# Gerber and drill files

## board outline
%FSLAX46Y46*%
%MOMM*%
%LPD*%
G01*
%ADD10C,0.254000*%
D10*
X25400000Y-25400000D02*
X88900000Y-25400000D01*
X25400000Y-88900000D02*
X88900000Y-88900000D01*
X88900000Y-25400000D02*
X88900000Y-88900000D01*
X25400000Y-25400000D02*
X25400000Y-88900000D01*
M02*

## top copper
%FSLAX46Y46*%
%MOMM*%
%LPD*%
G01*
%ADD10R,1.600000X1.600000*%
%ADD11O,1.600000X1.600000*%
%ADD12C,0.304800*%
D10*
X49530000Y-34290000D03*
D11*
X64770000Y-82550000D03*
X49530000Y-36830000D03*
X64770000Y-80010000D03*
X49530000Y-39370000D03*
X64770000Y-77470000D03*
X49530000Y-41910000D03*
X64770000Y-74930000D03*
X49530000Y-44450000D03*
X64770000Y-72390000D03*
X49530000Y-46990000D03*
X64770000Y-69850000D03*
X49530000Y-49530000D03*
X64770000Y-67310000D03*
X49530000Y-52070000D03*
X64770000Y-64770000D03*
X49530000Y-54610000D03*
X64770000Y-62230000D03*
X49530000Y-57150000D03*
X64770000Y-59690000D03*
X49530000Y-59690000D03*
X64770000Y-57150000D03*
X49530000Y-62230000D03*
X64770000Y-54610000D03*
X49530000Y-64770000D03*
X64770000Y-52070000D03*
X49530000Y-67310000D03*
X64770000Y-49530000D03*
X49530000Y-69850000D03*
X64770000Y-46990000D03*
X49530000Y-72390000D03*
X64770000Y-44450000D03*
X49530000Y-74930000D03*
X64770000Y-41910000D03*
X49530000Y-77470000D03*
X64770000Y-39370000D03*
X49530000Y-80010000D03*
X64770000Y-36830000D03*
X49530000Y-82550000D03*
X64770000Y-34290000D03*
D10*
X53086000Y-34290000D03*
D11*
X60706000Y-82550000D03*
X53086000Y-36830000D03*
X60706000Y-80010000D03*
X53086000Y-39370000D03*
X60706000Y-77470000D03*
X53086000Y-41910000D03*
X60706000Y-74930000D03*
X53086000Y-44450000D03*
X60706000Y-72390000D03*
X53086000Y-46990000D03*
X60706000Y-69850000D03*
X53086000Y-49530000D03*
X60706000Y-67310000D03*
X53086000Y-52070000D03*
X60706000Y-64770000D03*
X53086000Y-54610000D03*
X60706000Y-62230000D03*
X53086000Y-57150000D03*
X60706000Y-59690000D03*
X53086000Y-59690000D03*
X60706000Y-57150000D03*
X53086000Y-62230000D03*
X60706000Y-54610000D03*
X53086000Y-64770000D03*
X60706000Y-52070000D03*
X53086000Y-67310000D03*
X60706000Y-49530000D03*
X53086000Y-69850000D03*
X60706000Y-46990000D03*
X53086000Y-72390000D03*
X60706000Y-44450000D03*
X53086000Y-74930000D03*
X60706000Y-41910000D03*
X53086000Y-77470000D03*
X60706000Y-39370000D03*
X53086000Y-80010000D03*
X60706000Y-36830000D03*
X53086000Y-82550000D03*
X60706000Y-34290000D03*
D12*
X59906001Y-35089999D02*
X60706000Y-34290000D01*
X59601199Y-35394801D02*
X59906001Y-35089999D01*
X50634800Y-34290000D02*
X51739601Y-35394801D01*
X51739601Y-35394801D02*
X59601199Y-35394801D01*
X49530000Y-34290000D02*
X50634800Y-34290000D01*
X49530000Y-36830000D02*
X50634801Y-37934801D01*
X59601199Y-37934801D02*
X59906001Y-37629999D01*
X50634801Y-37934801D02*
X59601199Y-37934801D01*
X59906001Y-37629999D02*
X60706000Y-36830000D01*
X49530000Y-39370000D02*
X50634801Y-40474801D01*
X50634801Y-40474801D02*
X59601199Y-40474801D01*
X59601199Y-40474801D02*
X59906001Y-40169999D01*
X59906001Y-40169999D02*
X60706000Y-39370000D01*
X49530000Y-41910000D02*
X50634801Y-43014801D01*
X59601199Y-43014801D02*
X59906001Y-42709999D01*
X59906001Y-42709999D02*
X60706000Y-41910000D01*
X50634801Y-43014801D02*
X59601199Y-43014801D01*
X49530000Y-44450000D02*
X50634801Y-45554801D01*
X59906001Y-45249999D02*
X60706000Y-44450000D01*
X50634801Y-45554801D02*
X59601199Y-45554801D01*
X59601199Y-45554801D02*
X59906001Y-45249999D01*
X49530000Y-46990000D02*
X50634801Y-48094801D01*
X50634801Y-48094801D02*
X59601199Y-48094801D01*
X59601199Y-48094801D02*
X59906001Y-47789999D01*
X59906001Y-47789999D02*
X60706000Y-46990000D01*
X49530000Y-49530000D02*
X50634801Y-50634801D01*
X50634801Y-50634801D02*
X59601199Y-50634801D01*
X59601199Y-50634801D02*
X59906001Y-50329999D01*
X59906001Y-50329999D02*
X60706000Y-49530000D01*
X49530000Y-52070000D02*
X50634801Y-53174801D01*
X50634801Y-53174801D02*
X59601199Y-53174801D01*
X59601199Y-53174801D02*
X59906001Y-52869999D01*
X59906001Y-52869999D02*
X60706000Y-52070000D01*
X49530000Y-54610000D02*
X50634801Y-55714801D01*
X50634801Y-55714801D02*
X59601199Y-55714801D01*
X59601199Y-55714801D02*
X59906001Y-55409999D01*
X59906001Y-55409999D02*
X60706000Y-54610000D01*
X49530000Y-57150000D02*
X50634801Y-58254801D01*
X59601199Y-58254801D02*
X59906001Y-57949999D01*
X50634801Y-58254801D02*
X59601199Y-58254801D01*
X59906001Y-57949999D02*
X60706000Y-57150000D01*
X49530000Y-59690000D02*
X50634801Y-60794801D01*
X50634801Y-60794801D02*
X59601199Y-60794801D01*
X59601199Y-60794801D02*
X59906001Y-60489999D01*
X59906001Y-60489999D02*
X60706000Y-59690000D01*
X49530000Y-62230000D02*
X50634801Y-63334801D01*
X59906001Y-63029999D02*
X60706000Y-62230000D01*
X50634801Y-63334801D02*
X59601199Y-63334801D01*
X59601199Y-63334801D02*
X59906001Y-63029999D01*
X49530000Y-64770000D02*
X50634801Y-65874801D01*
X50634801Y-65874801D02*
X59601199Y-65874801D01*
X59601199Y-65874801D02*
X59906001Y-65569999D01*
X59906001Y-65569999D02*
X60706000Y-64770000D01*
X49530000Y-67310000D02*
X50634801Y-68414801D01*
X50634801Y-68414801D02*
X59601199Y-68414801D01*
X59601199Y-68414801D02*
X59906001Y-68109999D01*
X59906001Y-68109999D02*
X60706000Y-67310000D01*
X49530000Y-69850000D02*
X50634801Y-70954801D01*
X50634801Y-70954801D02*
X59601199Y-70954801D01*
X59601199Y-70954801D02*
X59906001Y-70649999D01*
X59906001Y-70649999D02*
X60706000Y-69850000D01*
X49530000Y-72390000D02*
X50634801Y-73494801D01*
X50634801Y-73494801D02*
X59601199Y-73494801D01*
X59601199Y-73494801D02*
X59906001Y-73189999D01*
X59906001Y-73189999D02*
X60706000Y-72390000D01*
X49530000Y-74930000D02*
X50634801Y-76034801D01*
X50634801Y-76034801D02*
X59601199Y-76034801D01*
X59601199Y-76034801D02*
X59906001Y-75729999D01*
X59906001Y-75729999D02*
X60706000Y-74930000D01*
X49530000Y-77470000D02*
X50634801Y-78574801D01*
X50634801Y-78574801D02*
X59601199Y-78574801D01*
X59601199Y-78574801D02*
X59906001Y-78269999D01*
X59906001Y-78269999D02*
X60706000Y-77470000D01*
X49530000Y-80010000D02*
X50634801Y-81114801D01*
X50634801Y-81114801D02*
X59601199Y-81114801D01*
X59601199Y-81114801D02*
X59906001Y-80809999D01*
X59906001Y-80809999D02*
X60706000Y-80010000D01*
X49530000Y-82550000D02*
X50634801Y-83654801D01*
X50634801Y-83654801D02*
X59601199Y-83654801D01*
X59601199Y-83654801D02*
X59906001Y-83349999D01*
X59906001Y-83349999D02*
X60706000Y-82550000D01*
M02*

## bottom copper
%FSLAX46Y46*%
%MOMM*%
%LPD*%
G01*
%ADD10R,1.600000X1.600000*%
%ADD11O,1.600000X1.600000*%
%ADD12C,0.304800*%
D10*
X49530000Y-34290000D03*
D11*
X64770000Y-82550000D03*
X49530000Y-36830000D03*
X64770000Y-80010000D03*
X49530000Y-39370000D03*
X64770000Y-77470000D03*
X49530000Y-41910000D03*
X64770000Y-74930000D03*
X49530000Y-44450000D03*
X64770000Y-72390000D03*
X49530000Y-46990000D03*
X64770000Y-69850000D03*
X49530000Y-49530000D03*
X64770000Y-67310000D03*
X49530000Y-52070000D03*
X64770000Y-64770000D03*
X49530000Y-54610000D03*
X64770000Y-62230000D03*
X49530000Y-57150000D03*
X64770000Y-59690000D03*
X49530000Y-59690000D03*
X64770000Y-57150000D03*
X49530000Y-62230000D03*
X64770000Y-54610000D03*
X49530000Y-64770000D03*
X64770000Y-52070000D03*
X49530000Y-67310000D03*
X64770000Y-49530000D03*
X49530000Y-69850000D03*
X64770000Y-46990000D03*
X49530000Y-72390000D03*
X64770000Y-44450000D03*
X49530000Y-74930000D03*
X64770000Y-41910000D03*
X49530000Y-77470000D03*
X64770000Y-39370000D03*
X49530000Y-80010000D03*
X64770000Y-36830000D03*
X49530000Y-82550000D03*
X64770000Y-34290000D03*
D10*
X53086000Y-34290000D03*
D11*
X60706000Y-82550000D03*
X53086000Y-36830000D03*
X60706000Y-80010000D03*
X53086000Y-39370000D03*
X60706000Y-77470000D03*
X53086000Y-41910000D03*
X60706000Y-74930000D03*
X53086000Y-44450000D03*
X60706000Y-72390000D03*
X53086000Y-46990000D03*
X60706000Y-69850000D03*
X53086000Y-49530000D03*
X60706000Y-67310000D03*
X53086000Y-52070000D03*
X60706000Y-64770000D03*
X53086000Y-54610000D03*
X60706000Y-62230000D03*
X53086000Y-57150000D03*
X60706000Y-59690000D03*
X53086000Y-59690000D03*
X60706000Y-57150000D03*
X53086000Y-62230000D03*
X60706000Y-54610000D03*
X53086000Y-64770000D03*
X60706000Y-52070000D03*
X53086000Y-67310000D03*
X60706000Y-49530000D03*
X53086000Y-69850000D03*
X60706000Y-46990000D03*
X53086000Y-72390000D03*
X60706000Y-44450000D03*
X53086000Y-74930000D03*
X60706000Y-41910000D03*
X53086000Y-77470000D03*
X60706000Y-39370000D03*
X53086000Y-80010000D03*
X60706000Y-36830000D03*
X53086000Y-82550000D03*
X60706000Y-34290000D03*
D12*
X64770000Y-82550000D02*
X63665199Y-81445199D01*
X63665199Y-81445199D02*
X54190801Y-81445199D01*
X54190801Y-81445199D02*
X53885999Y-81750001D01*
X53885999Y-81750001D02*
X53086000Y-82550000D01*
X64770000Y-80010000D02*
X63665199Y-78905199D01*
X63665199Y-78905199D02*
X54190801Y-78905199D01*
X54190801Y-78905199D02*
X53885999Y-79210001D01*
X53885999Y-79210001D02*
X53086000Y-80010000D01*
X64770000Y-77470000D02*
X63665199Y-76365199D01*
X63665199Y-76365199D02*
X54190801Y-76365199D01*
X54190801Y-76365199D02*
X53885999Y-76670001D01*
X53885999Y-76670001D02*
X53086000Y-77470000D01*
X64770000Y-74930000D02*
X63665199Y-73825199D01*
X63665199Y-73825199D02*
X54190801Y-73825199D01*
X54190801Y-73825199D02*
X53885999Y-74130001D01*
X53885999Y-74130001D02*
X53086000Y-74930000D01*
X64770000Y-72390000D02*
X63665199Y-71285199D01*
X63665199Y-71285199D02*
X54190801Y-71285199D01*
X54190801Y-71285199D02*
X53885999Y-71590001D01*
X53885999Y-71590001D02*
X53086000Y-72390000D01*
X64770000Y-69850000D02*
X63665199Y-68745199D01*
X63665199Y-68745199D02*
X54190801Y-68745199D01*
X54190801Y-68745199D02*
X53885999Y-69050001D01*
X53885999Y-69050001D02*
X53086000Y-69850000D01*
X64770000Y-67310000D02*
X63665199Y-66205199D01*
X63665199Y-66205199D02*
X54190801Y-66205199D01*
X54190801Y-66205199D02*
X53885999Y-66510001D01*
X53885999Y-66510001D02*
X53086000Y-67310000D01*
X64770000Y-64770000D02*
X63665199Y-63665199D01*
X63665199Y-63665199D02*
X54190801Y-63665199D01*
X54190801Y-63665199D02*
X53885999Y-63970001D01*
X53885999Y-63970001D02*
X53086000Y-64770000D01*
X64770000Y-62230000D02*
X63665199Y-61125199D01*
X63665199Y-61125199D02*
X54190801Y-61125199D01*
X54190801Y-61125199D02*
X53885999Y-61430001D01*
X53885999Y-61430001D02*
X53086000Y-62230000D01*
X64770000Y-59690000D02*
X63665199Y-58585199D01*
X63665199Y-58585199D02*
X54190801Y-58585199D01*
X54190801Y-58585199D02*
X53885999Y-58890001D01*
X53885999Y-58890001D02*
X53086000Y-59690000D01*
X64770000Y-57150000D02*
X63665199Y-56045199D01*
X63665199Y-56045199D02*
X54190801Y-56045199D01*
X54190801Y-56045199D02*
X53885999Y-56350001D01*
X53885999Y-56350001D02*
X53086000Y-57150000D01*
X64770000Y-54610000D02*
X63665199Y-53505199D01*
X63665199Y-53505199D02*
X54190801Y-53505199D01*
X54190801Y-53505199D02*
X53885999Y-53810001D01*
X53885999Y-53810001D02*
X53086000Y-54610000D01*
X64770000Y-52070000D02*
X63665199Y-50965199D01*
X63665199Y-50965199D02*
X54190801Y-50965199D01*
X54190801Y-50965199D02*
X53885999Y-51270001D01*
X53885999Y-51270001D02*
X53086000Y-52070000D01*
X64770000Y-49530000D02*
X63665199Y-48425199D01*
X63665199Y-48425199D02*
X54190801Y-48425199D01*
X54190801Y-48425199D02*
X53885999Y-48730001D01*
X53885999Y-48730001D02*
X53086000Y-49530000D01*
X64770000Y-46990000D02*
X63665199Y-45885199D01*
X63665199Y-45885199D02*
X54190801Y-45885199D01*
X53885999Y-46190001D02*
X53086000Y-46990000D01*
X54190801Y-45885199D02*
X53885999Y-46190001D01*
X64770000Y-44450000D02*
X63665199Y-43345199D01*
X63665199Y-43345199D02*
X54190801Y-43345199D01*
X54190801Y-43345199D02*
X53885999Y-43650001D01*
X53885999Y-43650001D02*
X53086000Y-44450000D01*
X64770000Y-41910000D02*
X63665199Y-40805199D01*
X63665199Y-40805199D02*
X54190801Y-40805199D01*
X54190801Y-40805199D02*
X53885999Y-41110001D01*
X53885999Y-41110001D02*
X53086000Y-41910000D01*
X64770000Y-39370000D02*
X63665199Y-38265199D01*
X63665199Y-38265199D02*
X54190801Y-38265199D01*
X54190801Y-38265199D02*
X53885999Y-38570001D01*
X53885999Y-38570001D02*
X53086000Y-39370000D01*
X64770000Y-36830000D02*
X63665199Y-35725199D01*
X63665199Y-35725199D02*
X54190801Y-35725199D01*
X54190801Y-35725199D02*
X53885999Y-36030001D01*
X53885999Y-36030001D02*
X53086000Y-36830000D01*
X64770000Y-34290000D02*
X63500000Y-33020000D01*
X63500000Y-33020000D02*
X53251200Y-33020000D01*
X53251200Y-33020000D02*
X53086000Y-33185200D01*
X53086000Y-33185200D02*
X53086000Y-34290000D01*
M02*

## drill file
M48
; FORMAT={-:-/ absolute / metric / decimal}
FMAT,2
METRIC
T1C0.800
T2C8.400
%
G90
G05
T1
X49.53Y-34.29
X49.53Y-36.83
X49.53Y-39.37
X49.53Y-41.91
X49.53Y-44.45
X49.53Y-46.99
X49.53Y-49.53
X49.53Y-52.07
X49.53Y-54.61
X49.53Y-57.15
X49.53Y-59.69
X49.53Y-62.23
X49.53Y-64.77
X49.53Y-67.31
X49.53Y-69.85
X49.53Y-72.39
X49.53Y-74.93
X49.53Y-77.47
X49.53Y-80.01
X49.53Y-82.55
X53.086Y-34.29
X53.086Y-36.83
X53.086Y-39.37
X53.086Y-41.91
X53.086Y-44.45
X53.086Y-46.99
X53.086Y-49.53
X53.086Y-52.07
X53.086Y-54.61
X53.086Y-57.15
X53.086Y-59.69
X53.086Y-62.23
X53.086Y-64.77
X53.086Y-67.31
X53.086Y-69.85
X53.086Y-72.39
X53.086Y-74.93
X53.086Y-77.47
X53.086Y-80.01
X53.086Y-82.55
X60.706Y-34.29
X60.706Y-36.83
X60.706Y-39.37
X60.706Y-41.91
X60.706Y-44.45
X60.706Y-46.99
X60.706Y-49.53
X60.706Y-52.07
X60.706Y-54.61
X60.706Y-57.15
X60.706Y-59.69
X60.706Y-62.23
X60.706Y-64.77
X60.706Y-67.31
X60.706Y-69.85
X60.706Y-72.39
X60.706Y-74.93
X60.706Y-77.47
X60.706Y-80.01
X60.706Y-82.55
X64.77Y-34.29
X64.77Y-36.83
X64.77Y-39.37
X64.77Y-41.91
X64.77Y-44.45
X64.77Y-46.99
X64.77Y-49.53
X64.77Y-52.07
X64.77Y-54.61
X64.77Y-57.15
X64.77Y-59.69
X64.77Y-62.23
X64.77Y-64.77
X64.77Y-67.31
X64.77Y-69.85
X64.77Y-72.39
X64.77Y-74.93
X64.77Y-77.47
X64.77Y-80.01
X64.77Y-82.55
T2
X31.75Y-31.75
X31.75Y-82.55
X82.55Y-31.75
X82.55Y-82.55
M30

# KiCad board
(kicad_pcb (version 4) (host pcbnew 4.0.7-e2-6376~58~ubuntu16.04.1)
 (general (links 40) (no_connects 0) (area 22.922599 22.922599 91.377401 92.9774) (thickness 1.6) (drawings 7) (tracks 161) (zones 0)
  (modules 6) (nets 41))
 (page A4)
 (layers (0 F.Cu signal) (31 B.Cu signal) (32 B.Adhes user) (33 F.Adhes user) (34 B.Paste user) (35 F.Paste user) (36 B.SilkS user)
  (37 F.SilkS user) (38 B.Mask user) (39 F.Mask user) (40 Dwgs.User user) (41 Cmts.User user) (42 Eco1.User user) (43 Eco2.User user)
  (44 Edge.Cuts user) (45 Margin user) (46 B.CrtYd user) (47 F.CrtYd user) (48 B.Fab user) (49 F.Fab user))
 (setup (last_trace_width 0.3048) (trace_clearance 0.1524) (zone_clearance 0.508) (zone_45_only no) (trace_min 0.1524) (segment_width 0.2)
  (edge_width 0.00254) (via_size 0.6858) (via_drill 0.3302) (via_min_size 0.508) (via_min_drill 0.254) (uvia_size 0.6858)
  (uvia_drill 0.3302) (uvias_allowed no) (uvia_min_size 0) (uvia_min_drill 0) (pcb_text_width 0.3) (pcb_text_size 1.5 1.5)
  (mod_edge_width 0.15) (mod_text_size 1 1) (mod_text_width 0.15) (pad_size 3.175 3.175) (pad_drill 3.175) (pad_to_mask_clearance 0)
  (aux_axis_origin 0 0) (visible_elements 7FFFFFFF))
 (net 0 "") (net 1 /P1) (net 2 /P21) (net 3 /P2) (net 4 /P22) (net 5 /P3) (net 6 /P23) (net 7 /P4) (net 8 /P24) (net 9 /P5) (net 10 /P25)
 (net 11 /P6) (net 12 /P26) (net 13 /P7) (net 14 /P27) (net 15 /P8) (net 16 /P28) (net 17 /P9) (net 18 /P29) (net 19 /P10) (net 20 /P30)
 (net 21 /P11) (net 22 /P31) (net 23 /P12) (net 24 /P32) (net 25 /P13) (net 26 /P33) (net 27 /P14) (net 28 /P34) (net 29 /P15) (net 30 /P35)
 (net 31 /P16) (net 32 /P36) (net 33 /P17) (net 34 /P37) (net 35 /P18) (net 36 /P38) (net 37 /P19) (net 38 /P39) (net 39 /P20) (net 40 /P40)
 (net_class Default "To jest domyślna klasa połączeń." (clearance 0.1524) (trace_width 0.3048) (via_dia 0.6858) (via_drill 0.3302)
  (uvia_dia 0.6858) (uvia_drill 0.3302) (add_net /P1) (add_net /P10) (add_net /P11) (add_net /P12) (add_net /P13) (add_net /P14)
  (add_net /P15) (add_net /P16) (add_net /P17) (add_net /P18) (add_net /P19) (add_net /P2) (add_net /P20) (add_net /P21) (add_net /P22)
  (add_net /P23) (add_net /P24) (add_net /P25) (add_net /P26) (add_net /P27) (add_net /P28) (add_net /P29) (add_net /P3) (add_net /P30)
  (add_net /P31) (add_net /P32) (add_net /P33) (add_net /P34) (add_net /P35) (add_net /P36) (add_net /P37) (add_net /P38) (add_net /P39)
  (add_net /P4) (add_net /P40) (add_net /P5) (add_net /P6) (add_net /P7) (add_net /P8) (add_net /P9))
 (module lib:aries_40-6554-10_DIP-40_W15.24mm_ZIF (layer F.Cu) (at 49.53 34.29)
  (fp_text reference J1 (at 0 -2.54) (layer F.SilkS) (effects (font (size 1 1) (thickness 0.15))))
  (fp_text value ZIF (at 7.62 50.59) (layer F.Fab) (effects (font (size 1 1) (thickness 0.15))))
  (pad 1 thru_hole rect (at 0 0) (size 1.6 1.6) (drill 0.8) (layers *.Cu *.Mask) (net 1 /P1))
  (pad 21 thru_hole oval (at 15.24 48.26) (size 1.6 1.6) (drill 0.8) (layers *.Cu *.Mask) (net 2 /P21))
  (pad 2 thru_hole oval (at 0 2.54) (size 1.6 1.6) (drill 0.8) (layers *.Cu *.Mask) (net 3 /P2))
  (pad 22 thru_hole oval (at 15.24 45.72) (size 1.6 1.6) (drill 0.8) (layers *.Cu *.Mask) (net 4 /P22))
  (pad 3 thru_hole oval (at 0 5.08) (size 1.6 1.6) (drill 0.8) (layers *.Cu *.Mask) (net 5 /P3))
  (pad 23 thru_hole oval (at 15.24 43.18) (size 1.6 1.6) (drill 0.8) (layers *.Cu *.Mask) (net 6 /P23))
  (pad 4 thru_hole oval (at 0 7.62) (size 1.6 1.6) (drill 0.8) (layers *.Cu *.Mask) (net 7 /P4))
  (pad 24 thru_hole oval (at 15.24 40.64) (size 1.6 1.6) (drill 0.8) (layers *.Cu *.Mask) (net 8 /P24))
  (pad 5 thru_hole oval (at 0 10.16) (size 1.6 1.6) (drill 0.8) (layers *.Cu *.Mask) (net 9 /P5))
  (pad 25 thru_hole oval (at 15.24 38.1) (size 1.6 1.6) (drill 0.8) (layers *.Cu *.Mask) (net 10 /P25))
  (pad 6 thru_hole oval (at 0 12.7) (size 1.6 1.6) (drill 0.8) (layers *.Cu *.Mask) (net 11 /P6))
  (pad 26 thru_hole oval (at 15.24 35.56) (size 1.6 1.6) (drill 0.8) (layers *.Cu *.Mask) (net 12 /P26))
  (pad 7 thru_hole oval (at 0 15.24) (size 1.6 1.6) (drill 0.8) (layers *.Cu *.Mask) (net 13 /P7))
  (pad 27 thru_hole oval (at 15.24 33.02) (size 1.6 1.6) (drill 0.8) (layers *.Cu *.Mask) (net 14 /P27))
  (pad 8 thru_hole oval (at 0 17.78) (size 1.6 1.6) (drill 0.8) (layers *.Cu *.Mask) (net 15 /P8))
  (pad 28 thru_hole oval (at 15.24 30.48) (size 1.6 1.6) (drill 0.8) (layers *.Cu *.Mask) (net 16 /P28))
  (pad 9 thru_hole oval (at 0 20.32) (size 1.6 1.6) (drill 0.8) (layers *.Cu *.Mask) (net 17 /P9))
  (pad 29 thru_hole oval (at 15.24 27.94) (size 1.6 1.6) (drill 0.8) (layers *.Cu *.Mask) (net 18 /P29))
  (pad 10 thru_hole oval (at 0 22.86) (size 1.6 1.6) (drill 0.8) (layers *.Cu *.Mask) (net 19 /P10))
  (pad 30 thru_hole oval (at 15.24 25.4) (size 1.6 1.6) (drill 0.8) (layers *.Cu *.Mask) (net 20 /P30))
  (pad 11 thru_hole oval (at 0 25.4) (size 1.6 1.6) (drill 0.8) (layers *.Cu *.Mask) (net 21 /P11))
  (pad 31 thru_hole oval (at 15.24 22.86) (size 1.6 1.6) (drill 0.8) (layers *.Cu *.Mask) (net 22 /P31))
  (pad 12 thru_hole oval (at 0 27.94) (size 1.6 1.6) (drill 0.8) (layers *.Cu *.Mask) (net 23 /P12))
  (pad 32 thru_hole oval (at 15.24 20.32) (size 1.6 1.6) (drill 0.8) (layers *.Cu *.Mask) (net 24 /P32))
  (pad 13 thru_hole oval (at 0 30.48) (size 1.6 1.6) (drill 0.8) (layers *.Cu *.Mask) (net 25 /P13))
  (pad 33 thru_hole oval (at 15.24 17.78) (size 1.6 1.6) (drill 0.8) (layers *.Cu *.Mask) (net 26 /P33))
  (pad 14 thru_hole oval (at 0 33.02) (size 1.6 1.6) (drill 0.8) (layers *.Cu *.Mask) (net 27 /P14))
  (pad 34 thru_hole oval (at 15.24 15.24) (size 1.6 1.6) (drill 0.8) (layers *.Cu *.Mask) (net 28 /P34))
  (pad 15 thru_hole oval (at 0 35.56) (size 1.6 1.6) (drill 0.8) (layers *.Cu *.Mask) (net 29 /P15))
  (pad 35 thru_hole oval (at 15.24 12.7) (size 1.6 1.6) (drill 0.8) (layers *.Cu *.Mask) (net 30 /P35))
  (pad 16 thru_hole oval (at 0 38.1) (size 1.6 1.6) (drill 0.8) (layers *.Cu *.Mask) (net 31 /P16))
  (pad 36 thru_hole oval (at 15.24 10.16) (size 1.6 1.6) (drill 0.8) (layers *.Cu *.Mask) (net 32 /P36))
  (pad 17 thru_hole oval (at 0 40.64) (size 1.6 1.6) (drill 0.8) (layers *.Cu *.Mask) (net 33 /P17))
  (pad 37 thru_hole oval (at 15.24 7.62) (size 1.6 1.6) (drill 0.8) (layers *.Cu *.Mask) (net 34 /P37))
  (pad 18 thru_hole oval (at 0 43.18) (size 1.6 1.6) (drill 0.8) (layers *.Cu *.Mask) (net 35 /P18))
  (pad 38 thru_hole oval (at 15.24 5.08) (size 1.6 1.6) (drill 0.8) (layers *.Cu *.Mask) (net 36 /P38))
  (pad 19 thru_hole oval (at 0 45.72) (size 1.6 1.6) (drill 0.8) (layers *.Cu *.Mask) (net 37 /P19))
  (pad 39 thru_hole oval (at 15.24 2.54) (size 1.6 1.6) (drill 0.8) (layers *.Cu *.Mask) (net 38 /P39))
  (pad 20 thru_hole oval (at 0 48.26) (size 1.6 1.6) (drill 0.8) (layers *.Cu *.Mask) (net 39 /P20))
  (pad 40 thru_hole oval (at 15.24 0) (size 1.6 1.6) (drill 0.8) (layers *.Cu *.Mask) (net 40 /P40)))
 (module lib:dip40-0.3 (layer F.Cu) (at 53.086 34.29)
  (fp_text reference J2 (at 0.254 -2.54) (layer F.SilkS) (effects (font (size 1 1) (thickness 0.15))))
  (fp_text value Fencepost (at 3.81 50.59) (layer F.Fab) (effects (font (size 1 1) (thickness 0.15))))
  (pad 1 thru_hole rect (at 0 0) (size 1.6 1.6) (drill 0.8) (layers *.Cu *.Mask) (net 40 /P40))
  (pad 21 thru_hole oval (at 7.62 48.26) (size 1.6 1.6) (drill 0.8) (layers *.Cu *.Mask) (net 39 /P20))
  (pad 2 thru_hole oval (at 0 2.54) (size 1.6 1.6) (drill 0.8) (layers *.Cu *.Mask) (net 38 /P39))
  (pad 22 thru_hole oval (at 7.62 45.72) (size 1.6 1.6) (drill 0.8) (layers *.Cu *.Mask) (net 37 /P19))
  (pad 3 thru_hole oval (at 0 5.08) (size 1.6 1.6) (drill 0.8) (layers *.Cu *.Mask) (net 36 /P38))
  (pad 23 thru_hole oval (at 7.62 43.18) (size 1.6 1.6) (drill 0.8) (layers *.Cu *.Mask) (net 35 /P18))
  (pad 4 thru_hole oval (at 0 7.62) (size 1.6 1.6) (drill 0.8) (layers *.Cu *.Mask) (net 34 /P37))
  (pad 24 thru_hole oval (at 7.62 40.64) (size 1.6 1.6) (drill 0.8) (layers *.Cu *.Mask) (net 33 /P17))
  (pad 5 thru_hole oval (at 0 10.16) (size 1.6 1.6) (drill 0.8) (layers *.Cu *.Mask) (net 32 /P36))
  (pad 25 thru_hole oval (at 7.62 38.1) (size 1.6 1.6) (drill 0.8) (layers *.Cu *.Mask) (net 31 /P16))
  (pad 6 thru_hole oval (at 0 12.7) (size 1.6 1.6) (drill 0.8) (layers *.Cu *.Mask) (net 30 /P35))
  (pad 26 thru_hole oval (at 7.62 35.56) (size 1.6 1.6) (drill 0.8) (layers *.Cu *.Mask) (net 29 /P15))
  (pad 7 thru_hole oval (at 0 15.24) (size 1.6 1.6) (drill 0.8) (layers *.Cu *.Mask) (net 28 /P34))
  (pad 27 thru_hole oval (at 7.62 33.02) (size 1.6 1.6) (drill 0.8) (layers *.Cu *.Mask) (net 27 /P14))
  (pad 8 thru_hole oval (at 0 17.78) (size 1.6 1.6) (drill 0.8) (layers *.Cu *.Mask) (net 26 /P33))
  (pad 28 thru_hole oval (at 7.62 30.48) (size 1.6 1.6) (drill 0.8) (layers *.Cu *.Mask) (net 25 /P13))
  (pad 9 thru_hole oval (at 0 20.32) (size 1.6 1.6) (drill 0.8) (layers *.Cu *.Mask) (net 24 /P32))
  (pad 29 thru_hole oval (at 7.62 27.94) (size 1.6 1.6) (drill 0.8) (layers *.Cu *.Mask) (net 23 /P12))
  (pad 10 thru_hole oval (at 0 22.86) (size 1.6 1.6) (drill 0.8) (layers *.Cu *.Mask) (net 22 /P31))
  (pad 30 thru_hole oval (at 7.62 25.4) (size 1.6 1.6) (drill 0.8) (layers *.Cu *.Mask) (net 21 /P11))
  (pad 11 thru_hole oval (at 0 25.4) (size 1.6 1.6) (drill 0.8) (layers *.Cu *.Mask) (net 20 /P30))
  (pad 31 thru_hole oval (at 7.62 22.86) (size 1.6 1.6) (drill 0.8) (layers *.Cu *.Mask) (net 19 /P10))
  (pad 12 thru_hole oval (at 0 27.94) (size 1.6 1.6) (drill 0.8) (layers *.Cu *.Mask) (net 18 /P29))
  (pad 32 thru_hole oval (at 7.62 20.32) (size 1.6 1.6) (drill 0.8) (layers *.Cu *.Mask) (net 17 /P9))
  (pad 13 thru_hole oval (at 0 30.48) (size 1.6 1.6) (drill 0.8) (layers *.Cu *.Mask) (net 16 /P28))
  (pad 33 thru_hole oval (at 7.62 17.78) (size 1.6 1.6) (drill 0.8) (layers *.Cu *.Mask) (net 15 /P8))
  (pad 14 thru_hole oval (at 0 33.02) (size 1.6 1.6) (drill 0.8) (layers *.Cu *.Mask) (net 14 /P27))
  (pad 34 thru_hole oval (at 7.62 15.24) (size 1.6 1.6) (drill 0.8) (layers *.Cu *.Mask) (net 13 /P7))
  (pad 15 thru_hole oval (at 0 35.56) (size 1.6 1.6) (drill 0.8) (layers *.Cu *.Mask) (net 12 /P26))
  (pad 35 thru_hole oval (at 7.62 12.7) (size 1.6 1.6) (drill 0.8) (layers *.Cu *.Mask) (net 11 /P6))
  (pad 16 thru_hole oval (at 0 38.1) (size 1.6 1.6) (drill 0.8) (layers *.Cu *.Mask) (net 10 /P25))
  (pad 36 thru_hole oval (at 7.62 10.16) (size 1.6 1.6) (drill 0.8) (layers *.Cu *.Mask) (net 9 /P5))
  (pad 17 thru_hole oval (at 0 40.64) (size 1.6 1.6) (drill 0.8) (layers *.Cu *.Mask) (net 8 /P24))
  (pad 37 thru_hole oval (at 7.62 7.62) (size 1.6 1.6) (drill 0.8) (layers *.Cu *.Mask) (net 7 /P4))
  (pad 18 thru_hole oval (at 0 43.18) (size 1.6 1.6) (drill 0.8) (layers *.Cu *.Mask) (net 6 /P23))
  (pad 38 thru_hole oval (at 7.62 5.08) (size 1.6 1.6) (drill 0.8) (layers *.Cu *.Mask) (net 5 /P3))
  (pad 19 thru_hole oval (at 0 45.72) (size 1.6 1.6) (drill 0.8) (layers *.Cu *.Mask) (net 4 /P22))
  (pad 39 thru_hole oval (at 7.62 2.54) (size 1.6 1.6) (drill 0.8) (layers *.Cu *.Mask) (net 3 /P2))
  (pad 20 thru_hole oval (at 0 48.26) (size 1.6 1.6) (drill 0.8) (layers *.Cu *.Mask) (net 2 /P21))
  (pad 40 thru_hole oval (at 7.62 0) (size 1.6 1.6) (drill 0.8) (layers *.Cu *.Mask) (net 1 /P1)))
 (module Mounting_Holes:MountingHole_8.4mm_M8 (layer F.Cu) (at 31.75 31.75)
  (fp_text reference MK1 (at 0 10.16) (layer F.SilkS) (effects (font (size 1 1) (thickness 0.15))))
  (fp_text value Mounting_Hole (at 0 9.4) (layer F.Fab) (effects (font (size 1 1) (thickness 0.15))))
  (pad 1 np_thru_hole circle (at 0 0) (size 8.4 8.4) (drill 8.4) (layers *.Cu *.Mask)))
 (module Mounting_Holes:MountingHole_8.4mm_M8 (layer F.Cu) (at 82.55 31.75)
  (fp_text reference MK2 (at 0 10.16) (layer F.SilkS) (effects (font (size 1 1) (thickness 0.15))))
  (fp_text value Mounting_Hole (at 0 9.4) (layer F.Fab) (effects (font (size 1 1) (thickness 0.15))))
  (pad 1 np_thru_hole circle (at 0 0) (size 8.4 8.4) (drill 8.4) (layers *.Cu *.Mask)))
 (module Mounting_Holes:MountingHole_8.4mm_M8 (layer F.Cu) (at 31.75 82.55)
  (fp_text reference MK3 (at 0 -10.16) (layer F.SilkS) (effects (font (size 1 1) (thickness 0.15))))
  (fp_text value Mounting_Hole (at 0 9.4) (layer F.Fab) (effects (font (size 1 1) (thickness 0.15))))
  (pad 1 np_thru_hole circle (at 0 0) (size 8.4 8.4) (drill 8.4) (layers *.Cu *.Mask)))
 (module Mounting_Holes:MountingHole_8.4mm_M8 (layer F.Cu) (at 82.55 82.55)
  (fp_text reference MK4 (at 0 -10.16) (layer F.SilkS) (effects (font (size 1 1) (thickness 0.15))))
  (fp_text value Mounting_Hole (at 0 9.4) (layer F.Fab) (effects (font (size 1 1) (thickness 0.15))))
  (pad 1 np_thru_hole circle (at 0 0) (size 8.4 8.4) (drill 8.4) (layers *.Cu *.Mask)))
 (gr_line (start 25.4 25.4) (end 88.9 25.4) (layer Edge.Cuts) (width 0.254))
 (gr_line (start 25.4 88.9) (end 88.9 88.9) (layer Edge.Cuts) (width 0.254))
 (gr_line (start 88.9 25.4) (end 88.9 88.9) (layer Edge.Cuts) (width 0.254))
 (gr_line (start 25.4 25.4) (end 25.4 88.9) (layer Edge.Cuts) (width 0.254))
 (segment (start 59.906001 35.089999) (end 60.706 34.29) (width 0.3048) (layer F.Cu) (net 1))
 (segment (start 59.601199 35.394801) (end 59.906001 35.089999) (width 0.3048) (layer F.Cu) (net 1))
 (segment (start 50.6348 34.29) (end 51.739601 35.394801) (width 0.3048) (layer F.Cu) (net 1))
 (segment (start 51.739601 35.394801) (end 59.601199 35.394801) (width 0.3048) (layer F.Cu) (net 1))
 (segment (start 49.53 34.29) (end 50.6348 34.29) (width 0.3048) (layer F.Cu) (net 1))
 (segment (start 64.77 82.55) (end 63.665199 81.445199) (width 0.3048) (layer B.Cu) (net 2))
 (segment (start 63.665199 81.445199) (end 54.190801 81.445199) (width 0.3048) (layer B.Cu) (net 2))
 (segment (start 54.190801 81.445199) (end 53.885999 81.750001) (width 0.3048) (layer B.Cu) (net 2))
 (segment (start 53.885999 81.750001) (end 53.086 82.55) (width 0.3048) (layer B.Cu) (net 2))
 (segment (start 49.53 36.83) (end 50.634801 37.934801) (width 0.3048) (layer F.Cu) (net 3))
 (segment (start 59.601199 37.934801) (end 59.906001 37.629999) (width 0.3048) (layer F.Cu) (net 3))
 (segment (start 50.634801 37.934801) (end 59.601199 37.934801) (width 0.3048) (layer F.Cu) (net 3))
 (segment (start 59.906001 37.629999) (end 60.706 36.83) (width 0.3048) (layer F.Cu) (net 3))
 (segment (start 64.77 80.01) (end 63.665199 78.905199) (width 0.3048) (layer B.Cu) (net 4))
 (segment (start 63.665199 78.905199) (end 54.190801 78.905199) (width 0.3048) (layer B.Cu) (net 4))
 (segment (start 54.190801 78.905199) (end 53.885999 79.210001) (width 0.3048) (layer B.Cu) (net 4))
 (segment (start 53.885999 79.210001) (end 53.086 80.01) (width 0.3048) (layer B.Cu) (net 4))
 (segment (start 49.53 39.37) (end 50.634801 40.474801) (width 0.3048) (layer F.Cu) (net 5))
 (segment (start 50.634801 40.474801) (end 59.601199 40.474801) (width 0.3048) (layer F.Cu) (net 5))
 (segment (start 59.601199 40.474801) (end 59.906001 40.169999) (width 0.3048) (layer F.Cu) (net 5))
 (segment (start 59.906001 40.169999) (end 60.706 39.37) (width 0.3048) (layer F.Cu) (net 5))
 (segment (start 64.77 77.47) (end 63.665199 76.365199) (width 0.3048) (layer B.Cu) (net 6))
 (segment (start 63.665199 76.365199) (end 54.190801 76.365199) (width 0.3048) (layer B.Cu) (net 6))
 (segment (start 54.190801 76.365199) (end 53.885999 76.670001) (width 0.3048) (layer B.Cu) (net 6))
 (segment (start 53.885999 76.670001) (end 53.086 77.47) (width 0.3048) (layer B.Cu) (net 6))
 (segment (start 49.53 41.91) (end 50.634801 43.014801) (width 0.3048) (layer F.Cu) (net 7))
 (segment (start 59.601199 43.014801) (end 59.906001 42.709999) (width 0.3048) (layer F.Cu) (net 7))
 (segment (start 59.906001 42.709999) (end 60.706 41.91) (width 0.3048) (layer F.Cu) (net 7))
 (segment (start 50.634801 43.014801) (end 59.601199 43.014801) (width 0.3048) (layer F.Cu) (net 7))
 (segment (start 64.77 74.93) (end 63.665199 73.825199) (width 0.3048) (layer B.Cu) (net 8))
 (segment (start 63.665199 73.825199) (end 54.190801 73.825199) (width 0.3048) (layer B.Cu) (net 8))
 (segment (start 54.190801 73.825199) (end 53.885999 74.130001) (width 0.3048) (layer B.Cu) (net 8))
 (segment (start 53.885999 74.130001) (end 53.086 74.93) (width 0.3048) (layer B.Cu) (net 8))
 (segment (start 49.53 44.45) (end 50.634801 45.554801) (width 0.3048) (layer F.Cu) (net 9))
 (segment (start 59.906001 45.249999) (end 60.706 44.45) (width 0.3048) (layer F.Cu) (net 9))
 (segment (start 50.634801 45.554801) (end 59.601199 45.554801) (width 0.3048) (layer F.Cu) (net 9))
 (segment (start 59.601199 45.554801) (end 59.906001 45.249999) (width 0.3048) (layer F.Cu) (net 9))
 (segment (start 64.77 72.39) (end 63.665199 71.285199) (width 0.3048) (layer B.Cu) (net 10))
 (segment (start 63.665199 71.285199) (end 54.190801 71.285199) (width 0.3048) (layer B.Cu) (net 10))
 (segment (start 54.190801 71.285199) (end 53.885999 71.590001) (width 0.3048) (layer B.Cu) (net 10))
 (segment (start 53.885999 71.590001) (end 53.086 72.39) (width 0.3048) (layer B.Cu) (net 10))
 (segment (start 49.53 46.99) (end 50.634801 48.094801) (width 0.3048) (layer F.Cu) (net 11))
 (segment (start 50.634801 48.094801) (end 59.601199 48.094801) (width 0.3048) (layer F.Cu) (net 11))
 (segment (start 59.601199 48.094801) (end 59.906001 47.789999) (width 0.3048) (layer F.Cu) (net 11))
 (segment (start 59.906001 47.789999) (end 60.706 46.99) (width 0.3048) (layer F.Cu) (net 11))
 (segment (start 64.77 69.85) (end 63.665199 68.745199) (width 0.3048) (layer B.Cu) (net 12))
 (segment (start 63.665199 68.745199) (end 54.190801 68.745199) (width 0.3048) (layer B.Cu) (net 12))
 (segment (start 54.190801 68.745199) (end 53.885999 69.050001) (width 0.3048) (layer B.Cu) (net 12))
 (segment (start 53.885999 69.050001) (end 53.086 69.85) (width 0.3048) (layer B.Cu) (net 12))
 (segment (start 49.53 49.53) (end 50.634801 50.634801) (width 0.3048) (layer F.Cu) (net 13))
 (segment (start 50.634801 50.634801) (end 59.601199 50.634801) (width 0.3048) (layer F.Cu) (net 13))
 (segment (start 59.601199 50.634801) (end 59.906001 50.329999) (width 0.3048) (layer F.Cu) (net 13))
 (segment (start 59.906001 50.329999) (end 60.706 49.53) (width 0.3048) (layer F.Cu) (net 13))
 (segment (start 64.77 67.31) (end 63.665199 66.205199) (width 0.3048) (layer B.Cu) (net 14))
 (segment (start 63.665199 66.205199) (end 54.190801 66.205199) (width 0.3048) (layer B.Cu) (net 14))
 (segment (start 54.190801 66.205199) (end 53.885999 66.510001) (width 0.3048) (layer B.Cu) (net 14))
 (segment (start 53.885999 66.510001) (end 53.086 67.31) (width 0.3048) (layer B.Cu) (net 14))
 (segment (start 49.53 52.07) (end 50.634801 53.174801) (width 0.3048) (layer F.Cu) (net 15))
 (segment (start 50.634801 53.174801) (end 59.601199 53.174801) (width 0.3048) (layer F.Cu) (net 15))
 (segment (start 59.601199 53.174801) (end 59.906001 52.869999) (width 0.3048) (layer F.Cu) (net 15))
 (segment (start 59.906001 52.869999) (end 60.706 52.07) (width 0.3048) (layer F.Cu) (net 15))
 (segment (start 64.77 64.77) (end 63.665199 63.665199) (width 0.3048) (layer B.Cu) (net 16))
 (segment (start 63.665199 63.665199) (end 54.190801 63.665199) (width 0.3048) (layer B.Cu) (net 16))
 (segment (start 54.190801 63.665199) (end 53.885999 63.970001) (width 0.3048) (layer B.Cu) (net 16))
 (segment (start 53.885999 63.970001) (end 53.086 64.77) (width 0.3048) (layer B.Cu) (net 16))
 (segment (start 49.53 54.61) (end 50.634801 55.714801) (width 0.3048) (layer F.Cu) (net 17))
 (segment (start 50.634801 55.714801) (end 59.601199 55.714801) (width 0.3048) (layer F.Cu) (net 17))
 (segment (start 59.601199 55.714801) (end 59.906001 55.409999) (width 0.3048) (layer F.Cu) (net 17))
 (segment (start 59.906001 55.409999) (end 60.706 54.61) (width 0.3048) (layer F.Cu) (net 17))
 (segment (start 64.77 62.23) (end 63.665199 61.125199) (width 0.3048) (layer B.Cu) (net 18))
 (segment (start 63.665199 61.125199) (end 54.190801 61.125199) (width 0.3048) (layer B.Cu) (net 18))
 (segment (start 54.190801 61.125199) (end 53.885999 61.430001) (width 0.3048) (layer B.Cu) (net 18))
 (segment (start 53.885999 61.430001) (end 53.086 62.23) (width 0.3048) (layer B.Cu) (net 18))
 (segment (start 49.53 57.15) (end 50.634801 58.254801) (width 0.3048) (layer F.Cu) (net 19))
 (segment (start 59.601199 58.254801) (end 59.906001 57.949999) (width 0.3048) (layer F.Cu) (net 19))
 (segment (start 50.634801 58.254801) (end 59.601199 58.254801) (width 0.3048) (layer F.Cu) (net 19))
 (segment (start 59.906001 57.949999) (end 60.706 57.15) (width 0.3048) (layer F.Cu) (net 19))
 (segment (start 64.77 59.69) (end 63.665199 58.585199) (width 0.3048) (layer B.Cu) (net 20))
 (segment (start 63.665199 58.585199) (end 54.190801 58.585199) (width 0.3048) (layer B.Cu) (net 20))
 (segment (start 54.190801 58.585199) (end 53.885999 58.890001) (width 0.3048) (layer B.Cu) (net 20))
 (segment (start 53.885999 58.890001) (end 53.086 59.69) (width 0.3048) (layer B.Cu) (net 20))
 (segment (start 49.53 59.69) (end 50.634801 60.794801) (width 0.3048) (layer F.Cu) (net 21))
 (segment (start 50.634801 60.794801) (end 59.601199 60.794801) (width 0.3048) (layer F.Cu) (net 21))
 (segment (start 59.601199 60.794801) (end 59.906001 60.489999) (width 0.3048) (layer F.Cu) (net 21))
 (segment (start 59.906001 60.489999) (end 60.706 59.69) (width 0.3048) (layer F.Cu) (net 21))
 (segment (start 64.77 57.15) (end 63.665199 56.045199) (width 0.3048) (layer B.Cu) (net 22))
 (segment (start 63.665199 56.045199) (end 54.190801 56.045199) (width 0.3048) (layer B.Cu) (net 22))
 (segment (start 54.190801 56.045199) (end 53.885999 56.350001) (width 0.3048) (layer B.Cu) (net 22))
 (segment (start 53.885999 56.350001) (end 53.086 57.15) (width 0.3048) (layer B.Cu) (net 22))
 (segment (start 49.53 62.23) (end 50.634801 63.334801) (width 0.3048) (layer F.Cu) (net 23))
 (segment (start 59.906001 63.029999) (end 60.706 62.23) (width 0.3048) (layer F.Cu) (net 23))
 (segment (start 50.634801 63.334801) (end 59.601199 63.334801) (width 0.3048) (layer F.Cu) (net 23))
 (segment (start 59.601199 63.334801) (end 59.906001 63.029999) (width 0.3048) (layer F.Cu) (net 23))
 (segment (start 64.77 54.61) (end 63.665199 53.505199) (width 0.3048) (layer B.Cu) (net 24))
 (segment (start 63.665199 53.505199) (end 54.190801 53.505199) (width 0.3048) (layer B.Cu) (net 24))
 (segment (start 54.190801 53.505199) (end 53.885999 53.810001) (width 0.3048) (layer B.Cu) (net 24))
 (segment (start 53.885999 53.810001) (end 53.086 54.61) (width 0.3048) (layer B.Cu) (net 24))
 (segment (start 49.53 64.77) (end 50.634801 65.874801) (width 0.3048) (layer F.Cu) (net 25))
 (segment (start 50.634801 65.874801) (end 59.601199 65.874801) (width 0.3048) (layer F.Cu) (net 25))
 (segment (start 59.601199 65.874801) (end 59.906001 65.569999) (width 0.3048) (layer F.Cu) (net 25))
 (segment (start 59.906001 65.569999) (end 60.706 64.77) (width 0.3048) (layer F.Cu) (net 25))
 (segment (start 64.77 52.07) (end 63.665199 50.965199) (width 0.3048) (layer B.Cu) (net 26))
 (segment (start 63.665199 50.965199) (end 54.190801 50.965199) (width 0.3048) (layer B.Cu) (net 26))
 (segment (start 54.190801 50.965199) (end 53.885999 51.270001) (width 0.3048) (layer B.Cu) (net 26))
 (segment (start 53.885999 51.270001) (end 53.086 52.07) (width 0.3048) (layer B.Cu) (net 26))
 (segment (start 49.53 67.31) (end 50.634801 68.414801) (width 0.3048) (layer F.Cu) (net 27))
 (segment (start 50.634801 68.414801) (end 59.601199 68.414801) (width 0.3048) (layer F.Cu) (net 27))
 (segment (start 59.601199 68.414801) (end 59.906001 68.109999) (width 0.3048) (layer F.Cu) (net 27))
 (segment (start 59.906001 68.109999) (end 60.706 67.31) (width 0.3048) (layer F.Cu) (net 27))
 (segment (start 64.77 49.53) (end 63.665199 48.425199) (width 0.3048) (layer B.Cu) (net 28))
 (segment (start 63.665199 48.425199) (end 54.190801 48.425199) (width 0.3048) (layer B.Cu) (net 28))
 (segment (start 54.190801 48.425199) (end 53.885999 48.730001) (width 0.3048) (layer B.Cu) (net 28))
 (segment (start 53.885999 48.730001) (end 53.086 49.53) (width 0.3048) (layer B.Cu) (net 28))
 (segment (start 49.53 69.85) (end 50.634801 70.954801) (width 0.3048) (layer F.Cu) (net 29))
 (segment (start 50.634801 70.954801) (end 59.601199 70.954801) (width 0.3048) (layer F.Cu) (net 29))
 (segment (start 59.601199 70.954801) (end 59.906001 70.649999) (width 0.3048) (layer F.Cu) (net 29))
 (segment (start 59.906001 70.649999) (end 60.706 69.85) (width 0.3048) (layer F.Cu) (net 29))
 (segment (start 64.77 46.99) (end 63.665199 45.885199) (width 0.3048) (layer B.Cu) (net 30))
 (segment (start 63.665199 45.885199) (end 54.190801 45.885199) (width 0.3048) (layer B.Cu) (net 30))
 (segment (start 53.885999 46.190001) (end 53.086 46.99) (width 0.3048) (layer B.Cu) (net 30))
 (segment (start 54.190801 45.885199) (end 53.885999 46.190001) (width 0.3048) (layer B.Cu) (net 30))
 (segment (start 49.53 72.39) (end 50.634801 73.494801) (width 0.3048) (layer F.Cu) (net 31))
 (segment (start 50.634801 73.494801) (end 59.601199 73.494801) (width 0.3048) (layer F.Cu) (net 31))
 (segment (start 59.601199 73.494801) (end 59.906001 73.189999) (width 0.3048) (layer F.Cu) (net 31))
 (segment (start 59.906001 73.189999) (end 60.706 72.39) (width 0.3048) (layer F.Cu) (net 31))
 (segment (start 64.77 44.45) (end 63.665199 43.345199) (width 0.3048) (layer B.Cu) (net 32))
 (segment (start 63.665199 43.345199) (end 54.190801 43.345199) (width 0.3048) (layer B.Cu) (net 32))
 (segment (start 54.190801 43.345199) (end 53.885999 43.650001) (width 0.3048) (layer B.Cu) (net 32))
 (segment (start 53.885999 43.650001) (end 53.086 44.45) (width 0.3048) (layer B.Cu) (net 32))
 (segment (start 49.53 74.93) (end 50.634801 76.034801) (width 0.3048) (layer F.Cu) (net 33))
 (segment (start 50.634801 76.034801) (end 59.601199 76.034801) (width 0.3048) (layer F.Cu) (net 33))
 (segment (start 59.601199 76.034801) (end 59.906001 75.729999) (width 0.3048) (layer F.Cu) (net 33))
 (segment (start 59.906001 75.729999) (end 60.706 74.93) (width 0.3048) (layer F.Cu) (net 33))
 (segment (start 64.77 41.91) (end 63.665199 40.805199) (width 0.3048) (layer B.Cu) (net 34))
 (segment (start 63.665199 40.805199) (end 54.190801 40.805199) (width 0.3048) (layer B.Cu) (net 34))
 (segment (start 54.190801 40.805199) (end 53.885999 41.110001) (width 0.3048) (layer B.Cu) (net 34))
 (segment (start 53.885999 41.110001) (end 53.086 41.91) (width 0.3048) (layer B.Cu) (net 34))
 (segment (start 49.53 77.47) (end 50.634801 78.574801) (width 0.3048) (layer F.Cu) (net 35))
 (segment (start 50.634801 78.574801) (end 59.601199 78.574801) (width 0.3048) (layer F.Cu) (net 35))
 (segment (start 59.601199 78.574801) (end 59.906001 78.269999) (width 0.3048) (layer F.Cu) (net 35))
 (segment (start 59.906001 78.269999) (end 60.706 77.47) (width 0.3048) (layer F.Cu) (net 35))
 (segment (start 64.77 39.37) (end 63.665199 38.265199) (width 0.3048) (layer B.Cu) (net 36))
 (segment (start 63.665199 38.265199) (end 54.190801 38.265199) (width 0.3048) (layer B.Cu) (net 36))
 (segment (start 54.190801 38.265199) (end 53.885999 38.570001) (width 0.3048) (layer B.Cu) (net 36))
 (segment (start 53.885999 38.570001) (end 53.086 39.37) (width 0.3048) (layer B.Cu) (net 36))
 (segment (start 49.53 80.01) (end 50.634801 81.114801) (width 0.3048) (layer F.Cu) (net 37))
 (segment (start 50.634801 81.114801) (end 59.601199 81.114801) (width 0.3048) (layer F.Cu) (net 37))
 (segment (start 59.601199 81.114801) (end 59.906001 80.809999) (width 0.3048) (layer F.Cu) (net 37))
 (segment (start 59.906001 80.809999) (end 60.706 80.01) (width 0.3048) (layer F.Cu) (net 37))
 (segment (start 64.77 36.83) (end 63.665199 35.725199) (width 0.3048) (layer B.Cu) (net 38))
 (segment (start 63.665199 35.725199) (end 54.190801 35.725199) (width 0.3048) (layer B.Cu) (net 38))
 (segment (start 54.190801 35.725199) (end 53.885999 36.030001) (width 0.3048) (layer B.Cu) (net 38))
 (segment (start 53.885999 36.030001) (end 53.086 36.83) (width 0.3048) (layer B.Cu) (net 38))
 (segment (start 49.53 82.55) (end 50.634801 83.654801) (width 0.3048) (layer F.Cu) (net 39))
 (segment (start 50.634801 83.654801) (end 59.601199 83.654801) (width 0.3048) (layer F.Cu) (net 39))
 (segment (start 59.601199 83.654801) (end 59.906001 83.349999) (width 0.3048) (layer F.Cu) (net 39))
 (segment (start 59.906001 83.349999) (end 60.706 82.55) (width 0.3048) (layer F.Cu) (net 39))
 (segment (start 64.77 34.29) (end 63.5 33.02) (width 0.3048) (layer B.Cu) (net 40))
 (segment (start 63.5 33.02) (end 53.2512 33.02) (width 0.3048) (layer B.Cu) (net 40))
 (segment (start 53.2512 33.02) (end 53.086 33.1852) (width 0.3048) (layer B.Cu) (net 40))
 (segment (start 53.086 33.1852) (end 53.086 34.29) (width 0.3048) (layer B.Cu) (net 40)))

